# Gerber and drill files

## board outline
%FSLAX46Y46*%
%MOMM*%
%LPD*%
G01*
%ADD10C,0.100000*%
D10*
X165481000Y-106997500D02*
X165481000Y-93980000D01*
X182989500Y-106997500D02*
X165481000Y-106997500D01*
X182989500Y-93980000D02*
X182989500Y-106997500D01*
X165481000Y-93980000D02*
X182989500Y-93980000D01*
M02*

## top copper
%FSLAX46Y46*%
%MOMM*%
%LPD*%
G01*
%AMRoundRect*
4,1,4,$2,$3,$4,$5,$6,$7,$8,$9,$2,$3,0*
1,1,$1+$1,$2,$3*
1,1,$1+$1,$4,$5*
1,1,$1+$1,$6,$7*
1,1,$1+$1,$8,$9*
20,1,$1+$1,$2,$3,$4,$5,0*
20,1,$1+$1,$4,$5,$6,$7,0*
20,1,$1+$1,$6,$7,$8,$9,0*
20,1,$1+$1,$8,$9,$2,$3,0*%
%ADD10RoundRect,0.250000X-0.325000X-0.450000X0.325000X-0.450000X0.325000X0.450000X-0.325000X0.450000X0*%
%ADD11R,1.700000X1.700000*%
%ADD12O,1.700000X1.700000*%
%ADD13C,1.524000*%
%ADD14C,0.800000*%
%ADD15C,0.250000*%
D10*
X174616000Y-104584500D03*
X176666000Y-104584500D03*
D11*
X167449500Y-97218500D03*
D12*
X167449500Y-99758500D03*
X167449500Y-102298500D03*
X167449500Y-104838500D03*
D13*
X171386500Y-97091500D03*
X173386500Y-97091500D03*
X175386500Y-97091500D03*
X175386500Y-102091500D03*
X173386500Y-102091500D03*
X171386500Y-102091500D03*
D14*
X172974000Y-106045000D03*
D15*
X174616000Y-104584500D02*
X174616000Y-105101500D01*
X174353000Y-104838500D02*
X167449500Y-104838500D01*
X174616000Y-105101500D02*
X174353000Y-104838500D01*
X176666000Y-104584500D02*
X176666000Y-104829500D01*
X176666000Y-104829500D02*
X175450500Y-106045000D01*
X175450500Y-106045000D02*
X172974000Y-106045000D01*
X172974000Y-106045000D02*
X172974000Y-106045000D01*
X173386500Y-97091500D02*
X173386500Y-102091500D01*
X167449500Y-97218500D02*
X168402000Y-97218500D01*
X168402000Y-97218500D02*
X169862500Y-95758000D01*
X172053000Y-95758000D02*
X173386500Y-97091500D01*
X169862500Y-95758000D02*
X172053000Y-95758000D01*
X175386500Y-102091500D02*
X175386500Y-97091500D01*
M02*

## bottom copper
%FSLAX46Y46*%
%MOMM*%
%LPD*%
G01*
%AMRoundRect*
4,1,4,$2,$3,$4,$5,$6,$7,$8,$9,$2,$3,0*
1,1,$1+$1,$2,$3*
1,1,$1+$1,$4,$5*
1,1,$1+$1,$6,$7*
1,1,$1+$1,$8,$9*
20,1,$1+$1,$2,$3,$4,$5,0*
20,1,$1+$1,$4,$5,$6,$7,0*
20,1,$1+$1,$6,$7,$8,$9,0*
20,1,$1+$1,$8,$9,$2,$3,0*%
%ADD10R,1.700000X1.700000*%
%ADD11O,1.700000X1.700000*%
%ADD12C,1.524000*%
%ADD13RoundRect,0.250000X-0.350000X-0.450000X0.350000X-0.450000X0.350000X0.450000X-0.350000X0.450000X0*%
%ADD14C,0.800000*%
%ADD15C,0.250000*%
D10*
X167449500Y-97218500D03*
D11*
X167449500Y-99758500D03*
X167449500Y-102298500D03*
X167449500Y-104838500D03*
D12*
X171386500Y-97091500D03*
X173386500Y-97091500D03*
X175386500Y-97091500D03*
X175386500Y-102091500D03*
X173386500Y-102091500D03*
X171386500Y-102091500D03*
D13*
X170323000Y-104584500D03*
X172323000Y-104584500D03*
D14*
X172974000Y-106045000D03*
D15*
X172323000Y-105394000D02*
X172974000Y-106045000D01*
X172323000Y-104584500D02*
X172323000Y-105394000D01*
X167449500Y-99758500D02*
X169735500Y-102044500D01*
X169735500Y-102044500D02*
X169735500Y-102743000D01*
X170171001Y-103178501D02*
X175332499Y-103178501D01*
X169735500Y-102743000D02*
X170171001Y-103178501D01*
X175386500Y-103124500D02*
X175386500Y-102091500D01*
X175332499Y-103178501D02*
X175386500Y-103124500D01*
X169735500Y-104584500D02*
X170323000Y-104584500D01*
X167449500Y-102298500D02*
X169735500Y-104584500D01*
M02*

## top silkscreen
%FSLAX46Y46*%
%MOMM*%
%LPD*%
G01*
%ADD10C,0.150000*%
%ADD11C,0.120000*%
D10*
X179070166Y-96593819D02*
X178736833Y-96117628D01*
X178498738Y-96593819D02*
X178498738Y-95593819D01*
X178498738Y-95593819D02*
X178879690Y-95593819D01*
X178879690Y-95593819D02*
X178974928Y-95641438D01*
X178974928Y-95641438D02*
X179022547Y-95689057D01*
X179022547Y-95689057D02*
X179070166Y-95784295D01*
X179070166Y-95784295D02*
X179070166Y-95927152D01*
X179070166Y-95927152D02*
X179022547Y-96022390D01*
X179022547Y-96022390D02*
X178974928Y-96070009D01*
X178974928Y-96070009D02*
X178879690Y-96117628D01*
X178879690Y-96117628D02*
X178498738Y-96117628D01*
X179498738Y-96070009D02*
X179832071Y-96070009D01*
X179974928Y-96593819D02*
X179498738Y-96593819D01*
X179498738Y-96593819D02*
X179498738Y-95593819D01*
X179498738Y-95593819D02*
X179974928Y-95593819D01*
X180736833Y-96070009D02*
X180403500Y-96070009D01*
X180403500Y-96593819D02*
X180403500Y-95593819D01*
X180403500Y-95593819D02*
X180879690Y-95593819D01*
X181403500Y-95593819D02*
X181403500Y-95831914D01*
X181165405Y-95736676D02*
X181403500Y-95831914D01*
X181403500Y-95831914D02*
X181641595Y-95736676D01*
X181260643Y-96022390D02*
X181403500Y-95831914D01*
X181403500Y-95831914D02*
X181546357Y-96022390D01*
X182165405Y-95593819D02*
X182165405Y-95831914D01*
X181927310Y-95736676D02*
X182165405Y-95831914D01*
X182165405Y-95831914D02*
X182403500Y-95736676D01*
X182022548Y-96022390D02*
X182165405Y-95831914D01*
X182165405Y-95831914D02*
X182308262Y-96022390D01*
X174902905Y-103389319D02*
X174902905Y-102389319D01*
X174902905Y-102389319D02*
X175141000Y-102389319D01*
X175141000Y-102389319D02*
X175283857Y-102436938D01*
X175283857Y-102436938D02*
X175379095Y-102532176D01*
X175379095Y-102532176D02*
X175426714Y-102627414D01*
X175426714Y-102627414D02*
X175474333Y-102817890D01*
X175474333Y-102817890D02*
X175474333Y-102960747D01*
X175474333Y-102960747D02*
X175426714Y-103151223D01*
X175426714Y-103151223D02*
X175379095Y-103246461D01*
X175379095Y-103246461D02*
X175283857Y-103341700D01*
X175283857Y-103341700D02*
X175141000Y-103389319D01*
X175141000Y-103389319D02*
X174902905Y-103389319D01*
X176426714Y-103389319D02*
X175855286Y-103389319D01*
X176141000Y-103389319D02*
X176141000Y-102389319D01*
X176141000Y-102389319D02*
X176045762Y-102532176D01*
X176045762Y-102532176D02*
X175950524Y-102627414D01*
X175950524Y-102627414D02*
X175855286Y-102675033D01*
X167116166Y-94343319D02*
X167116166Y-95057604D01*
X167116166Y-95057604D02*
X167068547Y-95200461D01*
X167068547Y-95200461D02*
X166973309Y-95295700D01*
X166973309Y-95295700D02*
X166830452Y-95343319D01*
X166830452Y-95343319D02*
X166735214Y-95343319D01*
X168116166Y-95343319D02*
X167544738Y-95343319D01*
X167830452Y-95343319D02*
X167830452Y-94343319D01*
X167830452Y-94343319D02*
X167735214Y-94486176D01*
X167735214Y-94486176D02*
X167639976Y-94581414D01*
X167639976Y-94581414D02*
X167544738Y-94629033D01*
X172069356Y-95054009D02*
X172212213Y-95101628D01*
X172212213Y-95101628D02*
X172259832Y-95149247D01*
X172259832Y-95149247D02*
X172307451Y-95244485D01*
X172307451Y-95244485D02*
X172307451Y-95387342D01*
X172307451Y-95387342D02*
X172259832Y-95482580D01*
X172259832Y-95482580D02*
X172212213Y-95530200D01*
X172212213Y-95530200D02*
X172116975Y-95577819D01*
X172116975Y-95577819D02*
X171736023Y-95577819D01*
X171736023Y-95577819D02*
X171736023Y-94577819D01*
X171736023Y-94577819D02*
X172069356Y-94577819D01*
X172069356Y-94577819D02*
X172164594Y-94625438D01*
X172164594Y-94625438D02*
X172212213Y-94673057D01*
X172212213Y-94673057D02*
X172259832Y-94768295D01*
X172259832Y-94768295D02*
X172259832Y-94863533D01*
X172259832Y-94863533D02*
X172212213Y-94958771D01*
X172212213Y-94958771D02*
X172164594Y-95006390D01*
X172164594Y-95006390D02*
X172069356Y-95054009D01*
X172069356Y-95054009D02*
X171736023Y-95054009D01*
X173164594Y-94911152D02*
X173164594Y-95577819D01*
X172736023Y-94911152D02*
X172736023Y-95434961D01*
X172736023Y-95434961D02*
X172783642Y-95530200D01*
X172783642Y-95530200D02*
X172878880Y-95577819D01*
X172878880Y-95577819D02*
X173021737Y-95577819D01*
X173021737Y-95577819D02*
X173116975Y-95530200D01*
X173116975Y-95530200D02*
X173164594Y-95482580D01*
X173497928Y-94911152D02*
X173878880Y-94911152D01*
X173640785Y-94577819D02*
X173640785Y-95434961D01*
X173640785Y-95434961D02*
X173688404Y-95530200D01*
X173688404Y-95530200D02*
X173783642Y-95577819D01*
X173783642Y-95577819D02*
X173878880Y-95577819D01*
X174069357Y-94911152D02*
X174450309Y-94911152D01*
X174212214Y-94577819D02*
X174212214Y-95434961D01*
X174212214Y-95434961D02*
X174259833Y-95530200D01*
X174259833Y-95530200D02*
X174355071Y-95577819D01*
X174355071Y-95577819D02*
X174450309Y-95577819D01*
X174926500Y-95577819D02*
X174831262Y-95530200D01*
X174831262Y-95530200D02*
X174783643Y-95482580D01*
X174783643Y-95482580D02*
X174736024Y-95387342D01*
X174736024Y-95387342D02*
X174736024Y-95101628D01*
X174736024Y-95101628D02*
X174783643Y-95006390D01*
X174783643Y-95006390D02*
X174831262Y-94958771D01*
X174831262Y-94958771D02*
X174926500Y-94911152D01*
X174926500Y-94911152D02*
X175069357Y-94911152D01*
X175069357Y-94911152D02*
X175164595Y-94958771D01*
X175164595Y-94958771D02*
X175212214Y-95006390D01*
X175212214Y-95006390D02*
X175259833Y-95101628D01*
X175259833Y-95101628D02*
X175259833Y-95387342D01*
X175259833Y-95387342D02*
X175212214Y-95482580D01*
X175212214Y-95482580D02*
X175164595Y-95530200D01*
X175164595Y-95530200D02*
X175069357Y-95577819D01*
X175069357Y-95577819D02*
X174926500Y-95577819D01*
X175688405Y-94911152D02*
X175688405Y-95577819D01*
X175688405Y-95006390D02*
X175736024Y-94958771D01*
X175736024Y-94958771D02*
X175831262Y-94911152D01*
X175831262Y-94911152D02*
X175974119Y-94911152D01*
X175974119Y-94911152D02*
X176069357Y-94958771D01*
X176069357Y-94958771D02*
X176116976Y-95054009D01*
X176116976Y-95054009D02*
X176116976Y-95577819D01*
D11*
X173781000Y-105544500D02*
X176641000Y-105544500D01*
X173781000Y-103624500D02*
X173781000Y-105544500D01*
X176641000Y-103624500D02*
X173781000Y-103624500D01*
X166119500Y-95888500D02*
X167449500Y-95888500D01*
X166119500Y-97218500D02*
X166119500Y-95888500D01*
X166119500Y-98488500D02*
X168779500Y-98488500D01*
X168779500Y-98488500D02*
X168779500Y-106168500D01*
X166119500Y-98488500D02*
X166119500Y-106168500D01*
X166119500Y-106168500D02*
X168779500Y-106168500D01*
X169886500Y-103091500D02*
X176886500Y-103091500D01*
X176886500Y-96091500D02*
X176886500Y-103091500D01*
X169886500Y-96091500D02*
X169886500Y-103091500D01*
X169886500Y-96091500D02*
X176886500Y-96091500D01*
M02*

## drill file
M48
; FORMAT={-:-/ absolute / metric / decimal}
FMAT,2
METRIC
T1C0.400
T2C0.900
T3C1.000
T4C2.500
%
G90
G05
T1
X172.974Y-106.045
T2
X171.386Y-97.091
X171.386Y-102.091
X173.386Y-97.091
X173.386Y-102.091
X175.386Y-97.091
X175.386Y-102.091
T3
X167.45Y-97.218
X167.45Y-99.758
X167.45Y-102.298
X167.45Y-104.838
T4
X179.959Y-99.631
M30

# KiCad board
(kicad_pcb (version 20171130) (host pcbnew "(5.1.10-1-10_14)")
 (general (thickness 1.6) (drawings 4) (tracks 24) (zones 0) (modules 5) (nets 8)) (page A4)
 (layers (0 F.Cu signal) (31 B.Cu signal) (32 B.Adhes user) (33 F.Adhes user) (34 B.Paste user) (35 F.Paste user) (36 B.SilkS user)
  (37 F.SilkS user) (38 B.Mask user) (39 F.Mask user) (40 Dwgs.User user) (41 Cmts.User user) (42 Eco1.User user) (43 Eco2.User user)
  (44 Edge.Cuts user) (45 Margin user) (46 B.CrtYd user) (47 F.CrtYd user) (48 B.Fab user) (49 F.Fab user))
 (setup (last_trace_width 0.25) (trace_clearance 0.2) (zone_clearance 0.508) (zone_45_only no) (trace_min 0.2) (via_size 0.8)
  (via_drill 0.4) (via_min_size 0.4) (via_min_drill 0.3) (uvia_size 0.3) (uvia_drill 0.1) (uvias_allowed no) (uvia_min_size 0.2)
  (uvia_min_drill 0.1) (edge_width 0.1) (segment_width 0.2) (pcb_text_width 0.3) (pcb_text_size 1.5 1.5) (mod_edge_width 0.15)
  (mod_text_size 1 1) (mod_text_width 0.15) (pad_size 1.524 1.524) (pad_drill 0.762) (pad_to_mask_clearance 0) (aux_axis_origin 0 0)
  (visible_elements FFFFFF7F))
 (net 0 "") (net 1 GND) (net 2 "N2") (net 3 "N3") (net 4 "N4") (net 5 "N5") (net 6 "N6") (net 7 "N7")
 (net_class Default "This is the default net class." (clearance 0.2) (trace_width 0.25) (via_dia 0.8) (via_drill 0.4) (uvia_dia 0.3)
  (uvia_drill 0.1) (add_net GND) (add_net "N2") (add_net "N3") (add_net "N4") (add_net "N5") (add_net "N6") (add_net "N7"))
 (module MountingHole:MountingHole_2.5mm (layer F.Cu) (at 179.959 99.6315)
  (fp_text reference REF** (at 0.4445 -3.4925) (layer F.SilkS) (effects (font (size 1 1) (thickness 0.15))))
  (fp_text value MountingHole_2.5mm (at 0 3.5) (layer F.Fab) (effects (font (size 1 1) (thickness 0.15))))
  (pad 1 np_thru_hole circle (at 0 0) (size 2.5 2.5) (drill 2.5) (layers *.Cu *.Mask)))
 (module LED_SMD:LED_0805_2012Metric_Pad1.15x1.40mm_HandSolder (layer F.Cu) (at 175.641 104.5845)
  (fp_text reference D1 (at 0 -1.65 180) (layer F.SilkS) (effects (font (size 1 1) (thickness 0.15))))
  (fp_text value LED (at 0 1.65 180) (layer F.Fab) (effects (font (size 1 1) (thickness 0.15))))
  (fp_line (start -1.86 0.96) (end 1 0.96) (layer F.SilkS) (width 0.12))
  (fp_line (start -1.86 -0.96) (end -1.86 0.96) (layer F.SilkS) (width 0.12))
  (fp_line (start 1 -0.96) (end -1.86 -0.96) (layer F.SilkS) (width 0.12))
  (pad 1 smd roundrect (at -1.025 0) (size 1.15 1.4) (layers F.Cu F.Paste F.Mask) (roundrect_rratio 0.217391) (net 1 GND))
  (pad 2 smd roundrect (at 1.025 0) (size 1.15 1.4) (layers F.Cu F.Paste F.Mask) (roundrect_rratio 0.217391) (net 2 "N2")))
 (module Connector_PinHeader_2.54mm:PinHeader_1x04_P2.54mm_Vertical (layer F.Cu) (at 167.4495 97.2185)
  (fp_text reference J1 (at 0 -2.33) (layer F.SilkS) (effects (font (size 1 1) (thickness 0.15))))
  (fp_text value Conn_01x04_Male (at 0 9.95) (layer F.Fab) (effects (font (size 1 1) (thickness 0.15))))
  (fp_line (start -1.33 -1.33) (end 0 -1.33) (layer F.SilkS) (width 0.12))
  (fp_line (start -1.33 0) (end -1.33 -1.33) (layer F.SilkS) (width 0.12))
  (fp_line (start -1.33 1.27) (end 1.33 1.27) (layer F.SilkS) (width 0.12))
  (fp_line (start 1.33 1.27) (end 1.33 8.95) (layer F.SilkS) (width 0.12))
  (fp_line (start -1.33 1.27) (end -1.33 8.95) (layer F.SilkS) (width 0.12))
  (fp_line (start -1.33 8.95) (end 1.33 8.95) (layer F.SilkS) (width 0.12))
  (pad 1 thru_hole rect (at 0 0) (size 1.7 1.7) (drill 1) (layers *.Cu *.Mask) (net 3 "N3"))
  (pad 2 thru_hole oval (at 0 2.54) (size 1.7 1.7) (drill 1) (layers *.Cu *.Mask) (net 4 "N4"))
  (pad 3 thru_hole oval (at 0 5.08) (size 1.7 1.7) (drill 1) (layers *.Cu *.Mask) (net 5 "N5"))
  (pad 4 thru_hole oval (at 0 7.62) (size 1.7 1.7) (drill 1) (layers *.Cu *.Mask) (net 1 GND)))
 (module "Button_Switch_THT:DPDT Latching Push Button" (layer F.Cu) (at 171.3865 97.0915)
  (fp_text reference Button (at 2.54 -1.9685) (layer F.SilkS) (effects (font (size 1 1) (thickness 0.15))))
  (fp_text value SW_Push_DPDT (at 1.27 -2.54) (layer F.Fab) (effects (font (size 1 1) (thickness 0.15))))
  (fp_line (start -1.5 6) (end 5.5 6) (layer F.SilkS) (width 0.12))
  (fp_line (start 5.5 -1) (end 5.5 6) (layer F.SilkS) (width 0.12))
  (fp_line (start -1.5 -1) (end -1.5 6) (layer F.SilkS) (width 0.12))
  (fp_line (start -1.5 -1) (end 5.5 -1) (layer F.SilkS) (width 0.12))
  (pad 1 thru_hole circle (at 0 0) (size 1.524 1.524) (drill 0.9) (layers *.Cu *.Mask) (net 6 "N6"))
  (pad 2 thru_hole circle (at 2 0) (size 1.524 1.524) (drill 0.9) (layers *.Cu *.Mask) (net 3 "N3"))
  (pad 3 thru_hole circle (at 4 0) (size 1.524 1.524) (drill 0.9) (layers *.Cu *.Mask) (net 4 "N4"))
  (pad 6 thru_hole circle (at 4 5) (size 1.524 1.524) (drill 0.9) (layers *.Cu *.Mask) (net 4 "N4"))
  (pad 5 thru_hole circle (at 2 5) (size 1.524 1.524) (drill 0.9) (layers *.Cu *.Mask) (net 3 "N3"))
  (pad 4 thru_hole circle (at 0 5) (size 1.524 1.524) (drill 0.9) (layers *.Cu *.Mask) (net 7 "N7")))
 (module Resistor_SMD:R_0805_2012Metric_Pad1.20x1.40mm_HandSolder (layer B.Cu) (at 171.323 104.5845)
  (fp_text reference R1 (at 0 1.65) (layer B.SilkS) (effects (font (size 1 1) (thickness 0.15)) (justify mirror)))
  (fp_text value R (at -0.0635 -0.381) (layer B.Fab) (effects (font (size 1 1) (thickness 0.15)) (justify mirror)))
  (pad 1 smd roundrect (at -1 0) (size 1.2 1.4) (layers B.Cu B.Paste B.Mask) (roundrect_rratio 0.208333) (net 5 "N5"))
  (pad 2 smd roundrect (at 1 0) (size 1.2 1.4) (layers B.Cu B.Paste B.Mask) (roundrect_rratio 0.208333) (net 2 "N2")))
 (gr_line (start 165.481 106.9975) (end 165.481 93.98) (layer Edge.Cuts) (width 0.1))
 (gr_line (start 182.9895 106.9975) (end 165.481 106.9975) (layer Edge.Cuts) (width 0.1))
 (gr_line (start 182.9895 93.98) (end 182.9895 106.9975) (layer Edge.Cuts) (width 0.1))
 (gr_line (start 165.481 93.98) (end 182.9895 93.98) (layer Edge.Cuts) (width 0.1))
 (segment (start 174.616 104.5845) (end 174.616 105.1015) (width 0.25) (layer F.Cu) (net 1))
 (segment (start 174.353 104.8385) (end 167.4495 104.8385) (width 0.25) (layer F.Cu) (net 1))
 (segment (start 174.616 105.1015) (end 174.353 104.8385) (width 0.25) (layer F.Cu) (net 1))
 (segment (start 176.666 104.5845) (end 176.666 104.8295) (width 0.25) (layer F.Cu) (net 2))
 (segment (start 176.666 104.8295) (end 175.4505 106.045) (width 0.25) (layer F.Cu) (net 2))
 (segment (start 175.4505 106.045) (end 172.974 106.045) (width 0.25) (layer F.Cu) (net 2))
 (segment (start 172.974 106.045) (end 172.974 106.045) (width 0.25) (layer F.Cu) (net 2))
 (via (at 172.974 106.045) (size 0.8) (drill 0.4) (layers F.Cu B.Cu) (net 2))
 (segment (start 172.323 105.394) (end 172.974 106.045) (width 0.25) (layer B.Cu) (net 2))
 (segment (start 172.323 104.5845) (end 172.323 105.394) (width 0.25) (layer B.Cu) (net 2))
 (segment (start 173.3865 97.0915) (end 173.3865 102.0915) (width 0.25) (layer F.Cu) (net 3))
 (segment (start 167.4495 97.2185) (end 168.402 97.2185) (width 0.25) (layer F.Cu) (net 3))
 (segment (start 168.402 97.2185) (end 169.8625 95.758) (width 0.25) (layer F.Cu) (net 3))
 (segment (start 172.053 95.758) (end 173.3865 97.0915) (width 0.25) (layer F.Cu) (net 3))
 (segment (start 169.8625 95.758) (end 172.053 95.758) (width 0.25) (layer F.Cu) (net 3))
 (segment (start 167.4495 99.7585) (end 169.7355 102.0445) (width 0.25) (layer B.Cu) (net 4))
 (segment (start 169.7355 102.0445) (end 169.7355 102.743) (width 0.25) (layer B.Cu) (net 4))
 (segment (start 170.171001 103.178501) (end 175.332499 103.178501) (width 0.25) (layer B.Cu) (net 4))
 (segment (start 169.7355 102.743) (end 170.171001 103.178501) (width 0.25) (layer B.Cu) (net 4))
 (segment (start 175.3865 103.1245) (end 175.3865 102.0915) (width 0.25) (layer B.Cu) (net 4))
 (segment (start 175.332499 103.178501) (end 175.3865 103.1245) (width 0.25) (layer B.Cu) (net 4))
 (segment (start 175.3865 102.0915) (end 175.3865 97.0915) (width 0.25) (layer F.Cu) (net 4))
 (segment (start 169.7355 104.5845) (end 170.323 104.5845) (width 0.25) (layer B.Cu) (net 5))
 (segment (start 167.4495 102.2985) (end 169.7355 104.5845) (width 0.25) (layer B.Cu) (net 5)))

